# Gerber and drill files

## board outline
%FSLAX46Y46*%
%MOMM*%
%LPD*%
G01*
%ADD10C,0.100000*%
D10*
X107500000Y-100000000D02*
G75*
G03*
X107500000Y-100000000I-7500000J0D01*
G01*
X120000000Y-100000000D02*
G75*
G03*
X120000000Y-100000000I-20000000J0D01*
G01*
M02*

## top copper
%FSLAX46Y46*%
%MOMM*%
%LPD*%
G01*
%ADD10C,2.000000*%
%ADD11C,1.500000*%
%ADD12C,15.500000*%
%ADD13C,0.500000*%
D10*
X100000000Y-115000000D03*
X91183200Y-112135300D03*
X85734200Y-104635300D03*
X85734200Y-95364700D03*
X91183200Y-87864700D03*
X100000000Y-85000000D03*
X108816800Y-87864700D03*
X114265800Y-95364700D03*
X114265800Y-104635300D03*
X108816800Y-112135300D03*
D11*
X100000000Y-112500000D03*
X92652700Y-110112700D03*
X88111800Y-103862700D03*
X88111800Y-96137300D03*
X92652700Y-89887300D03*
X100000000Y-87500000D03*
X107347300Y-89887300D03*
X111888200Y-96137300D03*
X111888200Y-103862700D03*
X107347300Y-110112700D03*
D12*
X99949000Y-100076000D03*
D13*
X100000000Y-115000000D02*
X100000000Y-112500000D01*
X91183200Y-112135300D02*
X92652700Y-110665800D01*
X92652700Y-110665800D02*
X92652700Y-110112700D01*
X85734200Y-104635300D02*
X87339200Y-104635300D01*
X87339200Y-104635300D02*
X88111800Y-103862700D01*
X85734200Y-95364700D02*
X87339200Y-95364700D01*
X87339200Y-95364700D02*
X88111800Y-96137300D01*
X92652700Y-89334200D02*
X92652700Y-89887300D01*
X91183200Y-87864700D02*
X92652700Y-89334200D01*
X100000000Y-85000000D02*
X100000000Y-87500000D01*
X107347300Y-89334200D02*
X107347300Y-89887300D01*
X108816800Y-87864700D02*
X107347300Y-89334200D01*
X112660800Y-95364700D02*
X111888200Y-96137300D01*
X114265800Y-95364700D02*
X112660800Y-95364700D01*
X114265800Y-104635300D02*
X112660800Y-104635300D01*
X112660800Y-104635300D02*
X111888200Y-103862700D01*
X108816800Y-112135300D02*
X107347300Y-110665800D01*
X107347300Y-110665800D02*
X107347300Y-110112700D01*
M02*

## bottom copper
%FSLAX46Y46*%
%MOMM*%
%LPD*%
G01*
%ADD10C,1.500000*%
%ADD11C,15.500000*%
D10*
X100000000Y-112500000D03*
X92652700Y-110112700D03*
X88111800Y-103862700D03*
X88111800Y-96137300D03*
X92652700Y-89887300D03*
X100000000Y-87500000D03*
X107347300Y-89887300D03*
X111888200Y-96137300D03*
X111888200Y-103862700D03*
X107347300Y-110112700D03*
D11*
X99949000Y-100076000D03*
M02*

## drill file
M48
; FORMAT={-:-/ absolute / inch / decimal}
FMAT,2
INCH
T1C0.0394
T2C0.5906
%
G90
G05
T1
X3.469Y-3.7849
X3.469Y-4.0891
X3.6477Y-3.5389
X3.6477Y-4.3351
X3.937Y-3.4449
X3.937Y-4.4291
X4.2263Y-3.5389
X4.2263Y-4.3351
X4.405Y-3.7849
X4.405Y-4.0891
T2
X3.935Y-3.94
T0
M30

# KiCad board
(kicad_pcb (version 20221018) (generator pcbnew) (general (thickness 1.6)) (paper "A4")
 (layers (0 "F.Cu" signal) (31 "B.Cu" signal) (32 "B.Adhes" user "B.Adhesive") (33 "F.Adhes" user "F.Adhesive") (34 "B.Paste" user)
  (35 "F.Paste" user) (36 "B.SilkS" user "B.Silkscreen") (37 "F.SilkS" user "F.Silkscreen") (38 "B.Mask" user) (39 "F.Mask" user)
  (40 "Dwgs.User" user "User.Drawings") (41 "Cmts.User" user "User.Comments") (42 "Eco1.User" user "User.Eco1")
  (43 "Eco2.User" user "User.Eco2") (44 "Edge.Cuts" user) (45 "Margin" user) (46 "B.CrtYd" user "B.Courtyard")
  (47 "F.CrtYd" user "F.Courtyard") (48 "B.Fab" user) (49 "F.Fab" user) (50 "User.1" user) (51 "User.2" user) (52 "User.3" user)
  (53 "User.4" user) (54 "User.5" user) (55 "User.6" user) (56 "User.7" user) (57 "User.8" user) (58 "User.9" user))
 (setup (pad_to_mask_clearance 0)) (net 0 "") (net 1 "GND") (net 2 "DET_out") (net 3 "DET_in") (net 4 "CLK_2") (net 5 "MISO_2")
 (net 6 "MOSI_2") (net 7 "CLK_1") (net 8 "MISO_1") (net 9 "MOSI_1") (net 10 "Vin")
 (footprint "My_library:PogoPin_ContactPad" (layer "F.Cu") (at 100 100)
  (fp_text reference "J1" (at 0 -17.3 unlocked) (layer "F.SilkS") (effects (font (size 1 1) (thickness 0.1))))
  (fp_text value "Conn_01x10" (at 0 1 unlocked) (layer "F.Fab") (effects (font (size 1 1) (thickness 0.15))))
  (pad "1" smd circle (at 0 15) (size 2 2) (layers "F.Cu" "F.Paste" "F.Mask") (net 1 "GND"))
  (pad "2" smd circle (at -8.8168 12.1353) (size 2 2) (layers "F.Cu" "F.Paste" "F.Mask") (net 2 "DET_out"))
  (pad "3" smd circle (at -14.2658 4.6353) (size 2 2) (layers "F.Cu" "F.Paste" "F.Mask") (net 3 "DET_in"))
  (pad "4" smd circle (at -14.2658 -4.6353) (size 2 2) (layers "F.Cu" "F.Paste" "F.Mask") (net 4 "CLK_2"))
  (pad "5" smd circle (at -8.8168 -12.1353) (size 2 2) (layers "F.Cu" "F.Paste" "F.Mask") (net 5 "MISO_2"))
  (pad "6" smd circle (at 0 -15) (size 2 2) (layers "F.Cu" "F.Paste" "F.Mask") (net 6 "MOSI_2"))
  (pad "7" smd circle (at 8.8168 -12.1353) (size 2 2) (layers "F.Cu" "F.Paste" "F.Mask") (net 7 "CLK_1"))
  (pad "8" smd circle (at 14.2658 -4.6353) (size 2 2) (layers "F.Cu" "F.Paste" "F.Mask") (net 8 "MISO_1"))
  (pad "9" smd circle (at 14.2658 4.6353) (size 2 2) (layers "F.Cu" "F.Paste" "F.Mask") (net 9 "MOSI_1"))
  (pad "10" smd circle (at 8.8168 12.1353) (size 2 2) (layers "F.Cu" "F.Paste" "F.Mask") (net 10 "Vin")))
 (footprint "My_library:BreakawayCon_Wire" (layer "F.Cu") (at 100 100)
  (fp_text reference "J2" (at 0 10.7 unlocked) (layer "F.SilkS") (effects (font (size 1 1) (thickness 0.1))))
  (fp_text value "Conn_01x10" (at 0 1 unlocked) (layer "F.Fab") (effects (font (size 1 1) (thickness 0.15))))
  (pad "1" thru_hole circle (at 0 12.5) (size 1.5 1.5) (drill 1) (layers "*.Cu" "*.Mask") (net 1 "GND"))
  (pad "2" thru_hole circle (at -7.3473 10.1127) (size 1.5 1.5) (drill 1) (layers "*.Cu" "*.Mask") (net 2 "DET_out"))
  (pad "3" thru_hole circle (at -11.8882 3.8627) (size 1.5 1.5) (drill 1) (layers "*.Cu" "*.Mask") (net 3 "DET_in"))
  (pad "4" thru_hole circle (at -11.8882 -3.8627) (size 1.5 1.5) (drill 1) (layers "*.Cu" "*.Mask") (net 4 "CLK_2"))
  (pad "5" thru_hole circle (at -7.3473 -10.1127) (size 1.5 1.5) (drill 1) (layers "*.Cu" "*.Mask") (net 5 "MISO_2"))
  (pad "6" thru_hole circle (at 0 -12.5) (size 1.5 1.5) (drill 1) (layers "*.Cu" "*.Mask") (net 6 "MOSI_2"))
  (pad "7" thru_hole circle (at 7.3473 -10.1127) (size 1.5 1.5) (drill 1) (layers "*.Cu" "*.Mask") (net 7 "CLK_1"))
  (pad "8" thru_hole circle (at 11.8882 -3.8627) (size 1.5 1.5) (drill 1) (layers "*.Cu" "*.Mask") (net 8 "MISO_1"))
  (pad "9" thru_hole circle (at 11.8882 3.8627) (size 1.5 1.5) (drill 1) (layers "*.Cu" "*.Mask") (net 9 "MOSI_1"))
  (pad "10" thru_hole circle (at 7.3473 10.1127) (size 1.5 1.5) (drill 1) (layers "*.Cu" "*.Mask") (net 10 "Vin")))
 (gr_circle (center 100 100) (end 107.5 100) (stroke (width 0.1) (type default)) (fill none) (layer "Edge.Cuts"))
 (gr_circle (center 100 100) (end 120 100) (stroke (width 0.1) (type default)) (fill none) (layer "Edge.Cuts"))
 (via (at 99.949 100.076) (size 15.5) (drill 15) (layers "F.Cu" "B.Cu") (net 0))
 (segment (start 100 115) (end 100 112.5) (width 0.5) (layer "F.Cu") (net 1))
 (segment (start 91.1832 112.1353) (end 92.6527 110.6658) (width 0.5) (layer "F.Cu") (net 2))
 (segment (start 92.6527 110.6658) (end 92.6527 110.1127) (width 0.5) (layer "F.Cu") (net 2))
 (segment (start 85.7342 104.6353) (end 87.3392 104.6353) (width 0.5) (layer "F.Cu") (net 3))
 (segment (start 87.3392 104.6353) (end 88.1118 103.8627) (width 0.5) (layer "F.Cu") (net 3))
 (segment (start 85.7342 95.3647) (end 87.3392 95.3647) (width 0.5) (layer "F.Cu") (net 4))
 (segment (start 87.3392 95.3647) (end 88.1118 96.1373) (width 0.5) (layer "F.Cu") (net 4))
 (segment (start 92.6527 89.3342) (end 92.6527 89.8873) (width 0.5) (layer "F.Cu") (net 5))
 (segment (start 91.1832 87.8647) (end 92.6527 89.3342) (width 0.5) (layer "F.Cu") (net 5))
 (segment (start 100 85) (end 100 87.5) (width 0.5) (layer "F.Cu") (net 6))
 (segment (start 107.3473 89.3342) (end 107.3473 89.8873) (width 0.5) (layer "F.Cu") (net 7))
 (segment (start 108.8168 87.8647) (end 107.3473 89.3342) (width 0.5) (layer "F.Cu") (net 7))
 (segment (start 112.6608 95.3647) (end 111.8882 96.1373) (width 0.5) (layer "F.Cu") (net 8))
 (segment (start 114.2658 95.3647) (end 112.6608 95.3647) (width 0.5) (layer "F.Cu") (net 8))
 (segment (start 114.2658 104.6353) (end 112.6608 104.6353) (width 0.5) (layer "F.Cu") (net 9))
 (segment (start 112.6608 104.6353) (end 111.8882 103.8627) (width 0.5) (layer "F.Cu") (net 9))
 (segment (start 108.8168 112.1353) (end 107.3473 110.6658) (width 0.5) (layer "F.Cu") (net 10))
 (segment (start 107.3473 110.6658) (end 107.3473 110.1127) (width 0.5) (layer "F.Cu") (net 10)))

